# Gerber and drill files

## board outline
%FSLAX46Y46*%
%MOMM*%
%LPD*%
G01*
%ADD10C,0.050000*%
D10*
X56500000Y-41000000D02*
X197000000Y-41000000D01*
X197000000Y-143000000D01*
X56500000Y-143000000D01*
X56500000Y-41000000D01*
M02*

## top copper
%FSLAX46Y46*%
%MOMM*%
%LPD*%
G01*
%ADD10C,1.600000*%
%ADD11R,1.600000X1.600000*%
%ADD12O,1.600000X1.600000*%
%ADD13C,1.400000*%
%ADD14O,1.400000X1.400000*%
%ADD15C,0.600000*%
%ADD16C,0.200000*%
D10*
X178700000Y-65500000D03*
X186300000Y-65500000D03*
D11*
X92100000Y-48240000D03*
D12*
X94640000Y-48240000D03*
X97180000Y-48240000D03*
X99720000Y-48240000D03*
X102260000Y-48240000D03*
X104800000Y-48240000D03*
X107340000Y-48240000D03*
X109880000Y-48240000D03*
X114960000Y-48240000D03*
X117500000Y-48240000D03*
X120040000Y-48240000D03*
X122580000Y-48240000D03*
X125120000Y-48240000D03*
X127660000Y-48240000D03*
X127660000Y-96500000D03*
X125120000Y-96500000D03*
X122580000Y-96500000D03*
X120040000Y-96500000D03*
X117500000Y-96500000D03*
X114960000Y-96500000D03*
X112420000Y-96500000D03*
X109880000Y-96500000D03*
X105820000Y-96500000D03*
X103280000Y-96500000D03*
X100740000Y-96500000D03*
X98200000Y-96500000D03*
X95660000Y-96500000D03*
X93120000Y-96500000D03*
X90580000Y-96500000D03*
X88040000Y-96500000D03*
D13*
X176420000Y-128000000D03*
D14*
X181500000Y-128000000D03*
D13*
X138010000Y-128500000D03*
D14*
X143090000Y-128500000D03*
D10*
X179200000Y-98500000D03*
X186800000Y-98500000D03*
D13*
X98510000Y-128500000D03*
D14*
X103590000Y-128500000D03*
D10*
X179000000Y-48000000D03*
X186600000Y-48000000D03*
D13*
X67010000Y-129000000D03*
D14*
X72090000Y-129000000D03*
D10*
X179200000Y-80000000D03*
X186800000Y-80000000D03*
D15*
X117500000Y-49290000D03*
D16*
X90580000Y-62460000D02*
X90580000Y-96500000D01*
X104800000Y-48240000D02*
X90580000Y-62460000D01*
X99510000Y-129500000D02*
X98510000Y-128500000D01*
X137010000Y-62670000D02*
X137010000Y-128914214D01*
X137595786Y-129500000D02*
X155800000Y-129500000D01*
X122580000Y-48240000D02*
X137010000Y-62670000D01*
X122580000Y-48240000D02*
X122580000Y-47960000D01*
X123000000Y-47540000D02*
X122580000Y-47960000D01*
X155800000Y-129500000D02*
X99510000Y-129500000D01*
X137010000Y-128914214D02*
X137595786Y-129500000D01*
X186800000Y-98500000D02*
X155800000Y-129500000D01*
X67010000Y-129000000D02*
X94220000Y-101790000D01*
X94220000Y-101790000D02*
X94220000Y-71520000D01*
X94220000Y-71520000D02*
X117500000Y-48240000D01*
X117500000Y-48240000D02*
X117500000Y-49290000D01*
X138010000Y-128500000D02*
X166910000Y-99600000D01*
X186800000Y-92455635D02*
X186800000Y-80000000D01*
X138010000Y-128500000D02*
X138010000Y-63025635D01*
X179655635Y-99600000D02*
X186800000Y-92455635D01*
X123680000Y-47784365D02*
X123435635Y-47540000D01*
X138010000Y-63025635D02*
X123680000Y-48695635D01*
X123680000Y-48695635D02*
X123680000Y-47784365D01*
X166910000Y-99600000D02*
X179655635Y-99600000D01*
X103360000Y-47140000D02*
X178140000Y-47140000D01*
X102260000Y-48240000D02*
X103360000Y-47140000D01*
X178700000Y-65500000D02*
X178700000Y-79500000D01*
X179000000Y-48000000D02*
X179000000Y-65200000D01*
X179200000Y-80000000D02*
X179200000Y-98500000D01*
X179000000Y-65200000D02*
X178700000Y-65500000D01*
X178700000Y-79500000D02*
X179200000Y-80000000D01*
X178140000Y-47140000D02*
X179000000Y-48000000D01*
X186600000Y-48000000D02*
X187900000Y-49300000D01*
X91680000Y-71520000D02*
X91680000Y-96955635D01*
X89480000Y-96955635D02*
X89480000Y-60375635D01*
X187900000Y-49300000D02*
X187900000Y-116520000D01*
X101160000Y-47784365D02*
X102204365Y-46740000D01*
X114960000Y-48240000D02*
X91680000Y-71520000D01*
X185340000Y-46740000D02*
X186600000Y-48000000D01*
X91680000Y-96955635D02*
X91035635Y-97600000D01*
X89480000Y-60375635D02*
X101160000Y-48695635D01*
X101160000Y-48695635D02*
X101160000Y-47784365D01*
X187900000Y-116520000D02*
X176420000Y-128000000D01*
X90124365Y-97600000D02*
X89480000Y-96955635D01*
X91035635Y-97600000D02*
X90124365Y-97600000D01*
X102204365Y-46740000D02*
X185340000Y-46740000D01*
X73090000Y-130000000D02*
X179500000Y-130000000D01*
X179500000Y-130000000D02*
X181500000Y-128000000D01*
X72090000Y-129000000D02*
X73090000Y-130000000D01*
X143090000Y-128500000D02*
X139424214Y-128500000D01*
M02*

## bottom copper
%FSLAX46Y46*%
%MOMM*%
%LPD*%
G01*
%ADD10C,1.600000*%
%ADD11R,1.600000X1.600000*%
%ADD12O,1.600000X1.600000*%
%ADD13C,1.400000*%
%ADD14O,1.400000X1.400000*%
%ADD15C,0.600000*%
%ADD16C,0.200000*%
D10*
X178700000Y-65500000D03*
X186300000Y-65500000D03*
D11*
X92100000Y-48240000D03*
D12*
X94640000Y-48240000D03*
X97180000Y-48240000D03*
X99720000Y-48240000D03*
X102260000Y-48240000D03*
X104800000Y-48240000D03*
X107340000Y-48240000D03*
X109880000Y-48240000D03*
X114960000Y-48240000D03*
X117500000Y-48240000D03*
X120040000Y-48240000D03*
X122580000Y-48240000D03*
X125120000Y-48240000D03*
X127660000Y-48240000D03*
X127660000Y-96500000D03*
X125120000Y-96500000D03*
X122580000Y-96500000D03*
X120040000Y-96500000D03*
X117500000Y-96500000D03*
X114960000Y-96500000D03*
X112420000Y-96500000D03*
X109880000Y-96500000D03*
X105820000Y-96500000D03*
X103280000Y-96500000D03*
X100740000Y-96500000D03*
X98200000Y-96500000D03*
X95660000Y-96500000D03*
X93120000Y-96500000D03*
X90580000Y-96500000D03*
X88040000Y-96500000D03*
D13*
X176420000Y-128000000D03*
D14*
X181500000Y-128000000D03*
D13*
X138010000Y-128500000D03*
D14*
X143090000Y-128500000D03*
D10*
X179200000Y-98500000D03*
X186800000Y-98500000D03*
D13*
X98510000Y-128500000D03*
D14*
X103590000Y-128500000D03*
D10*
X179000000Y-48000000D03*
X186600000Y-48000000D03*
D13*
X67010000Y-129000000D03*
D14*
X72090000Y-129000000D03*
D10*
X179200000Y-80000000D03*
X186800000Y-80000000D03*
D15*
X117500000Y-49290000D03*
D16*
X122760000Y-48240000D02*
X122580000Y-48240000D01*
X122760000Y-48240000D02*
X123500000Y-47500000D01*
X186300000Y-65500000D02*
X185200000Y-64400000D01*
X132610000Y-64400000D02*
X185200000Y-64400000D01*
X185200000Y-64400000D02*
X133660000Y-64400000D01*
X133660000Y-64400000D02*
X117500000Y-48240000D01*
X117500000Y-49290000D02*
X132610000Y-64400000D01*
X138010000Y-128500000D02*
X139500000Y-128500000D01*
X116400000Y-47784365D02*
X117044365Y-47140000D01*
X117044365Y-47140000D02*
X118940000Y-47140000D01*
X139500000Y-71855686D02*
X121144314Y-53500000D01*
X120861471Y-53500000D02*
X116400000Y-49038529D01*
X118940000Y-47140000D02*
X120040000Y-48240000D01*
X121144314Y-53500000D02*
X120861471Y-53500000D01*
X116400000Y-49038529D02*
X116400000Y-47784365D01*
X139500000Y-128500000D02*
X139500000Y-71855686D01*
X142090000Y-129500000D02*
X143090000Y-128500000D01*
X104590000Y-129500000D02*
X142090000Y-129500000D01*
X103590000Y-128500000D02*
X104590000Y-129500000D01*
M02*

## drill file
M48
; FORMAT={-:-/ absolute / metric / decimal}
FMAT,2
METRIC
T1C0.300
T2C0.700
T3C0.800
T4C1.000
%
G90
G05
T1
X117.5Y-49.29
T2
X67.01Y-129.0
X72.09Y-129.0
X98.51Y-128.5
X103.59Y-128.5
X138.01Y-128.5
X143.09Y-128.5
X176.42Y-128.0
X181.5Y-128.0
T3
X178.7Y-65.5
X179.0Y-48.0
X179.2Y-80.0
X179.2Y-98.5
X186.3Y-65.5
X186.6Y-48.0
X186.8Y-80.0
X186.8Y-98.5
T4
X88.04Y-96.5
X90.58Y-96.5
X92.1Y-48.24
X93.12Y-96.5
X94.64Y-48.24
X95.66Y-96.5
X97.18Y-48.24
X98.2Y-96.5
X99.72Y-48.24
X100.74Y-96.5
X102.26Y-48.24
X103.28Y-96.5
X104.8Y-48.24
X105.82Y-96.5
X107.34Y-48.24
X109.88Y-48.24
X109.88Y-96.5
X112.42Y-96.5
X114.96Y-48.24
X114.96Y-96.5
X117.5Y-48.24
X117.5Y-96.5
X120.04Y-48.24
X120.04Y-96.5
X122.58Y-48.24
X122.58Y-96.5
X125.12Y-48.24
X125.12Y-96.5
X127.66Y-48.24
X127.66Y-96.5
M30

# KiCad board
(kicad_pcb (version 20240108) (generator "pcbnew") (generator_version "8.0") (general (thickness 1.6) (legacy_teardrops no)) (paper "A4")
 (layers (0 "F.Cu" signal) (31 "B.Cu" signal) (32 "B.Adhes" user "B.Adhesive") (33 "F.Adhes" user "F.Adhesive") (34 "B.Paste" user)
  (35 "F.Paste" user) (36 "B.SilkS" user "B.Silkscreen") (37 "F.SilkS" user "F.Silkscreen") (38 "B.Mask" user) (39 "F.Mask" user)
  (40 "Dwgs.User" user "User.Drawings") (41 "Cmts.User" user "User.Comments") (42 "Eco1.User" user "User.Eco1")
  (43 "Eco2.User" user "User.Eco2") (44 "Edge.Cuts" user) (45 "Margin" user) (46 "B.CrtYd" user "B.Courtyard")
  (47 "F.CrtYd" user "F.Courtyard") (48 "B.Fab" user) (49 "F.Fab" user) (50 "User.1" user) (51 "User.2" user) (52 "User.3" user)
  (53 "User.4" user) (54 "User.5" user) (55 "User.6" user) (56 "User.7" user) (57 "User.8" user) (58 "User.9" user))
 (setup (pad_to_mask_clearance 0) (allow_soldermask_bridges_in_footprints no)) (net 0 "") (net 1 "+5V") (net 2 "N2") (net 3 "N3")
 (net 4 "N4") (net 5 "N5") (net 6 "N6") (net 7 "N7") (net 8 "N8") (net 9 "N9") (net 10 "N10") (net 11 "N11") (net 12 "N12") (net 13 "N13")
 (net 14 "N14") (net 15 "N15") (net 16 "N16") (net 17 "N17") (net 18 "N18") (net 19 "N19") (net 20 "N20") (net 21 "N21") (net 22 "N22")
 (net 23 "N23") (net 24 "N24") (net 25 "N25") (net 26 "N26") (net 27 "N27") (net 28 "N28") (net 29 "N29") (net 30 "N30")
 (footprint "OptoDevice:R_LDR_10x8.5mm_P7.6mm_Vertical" (layer "F.Cu") (at 178.7 65.5)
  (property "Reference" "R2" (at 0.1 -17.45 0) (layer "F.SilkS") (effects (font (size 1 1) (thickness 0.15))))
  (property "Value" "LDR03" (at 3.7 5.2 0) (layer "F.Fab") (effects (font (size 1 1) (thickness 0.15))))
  (pad "1" thru_hole circle (at 0 0) (size 1.6 1.6) (drill 0.8) (layers "*.Cu" "*.Mask") (remove_unused_layers no) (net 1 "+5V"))
  (pad "2" thru_hole circle (at 7.6 0) (size 1.6 1.6) (drill 0.8) (layers "*.Cu" "*.Mask") (remove_unused_layers no) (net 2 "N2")))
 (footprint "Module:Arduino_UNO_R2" (layer "F.Cu") (at 92.1 48.24)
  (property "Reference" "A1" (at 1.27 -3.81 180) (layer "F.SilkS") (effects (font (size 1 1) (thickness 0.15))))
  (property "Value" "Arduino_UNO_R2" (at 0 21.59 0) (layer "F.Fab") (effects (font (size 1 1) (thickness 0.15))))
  (pad "1" thru_hole rect (at 0 0 90) (size 1.6 1.6) (drill 1) (layers "*.Cu" "*.Mask") (remove_unused_layers no) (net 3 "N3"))
  (pad "2" thru_hole oval (at 2.54 0 90) (size 1.6 1.6) (drill 1) (layers "*.Cu" "*.Mask") (remove_unused_layers no) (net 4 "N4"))
  (pad "3" thru_hole oval (at 5.08 0 90) (size 1.6 1.6) (drill 1) (layers "*.Cu" "*.Mask") (remove_unused_layers no) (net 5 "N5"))
  (pad "4" thru_hole oval (at 7.62 0 90) (size 1.6 1.6) (drill 1) (layers "*.Cu" "*.Mask") (remove_unused_layers no) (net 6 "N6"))
  (pad "5" thru_hole oval (at 10.16 0 90) (size 1.6 1.6) (drill 1) (layers "*.Cu" "*.Mask") (remove_unused_layers no) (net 1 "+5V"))
  (pad "6" thru_hole oval (at 12.7 0 90) (size 1.6 1.6) (drill 1) (layers "*.Cu" "*.Mask") (remove_unused_layers no) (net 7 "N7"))
  (pad "7" thru_hole oval (at 15.24 0 90) (size 1.6 1.6) (drill 1) (layers "*.Cu" "*.Mask") (remove_unused_layers no) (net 7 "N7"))
  (pad "8" thru_hole oval (at 17.78 0 90) (size 1.6 1.6) (drill 1) (layers "*.Cu" "*.Mask") (remove_unused_layers no) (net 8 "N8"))
  (pad "9" thru_hole oval (at 22.86 0 90) (size 1.6 1.6) (drill 1) (layers "*.Cu" "*.Mask") (remove_unused_layers no) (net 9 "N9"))
  (pad "10" thru_hole oval (at 25.4 0 90) (size 1.6 1.6) (drill 1) (layers "*.Cu" "*.Mask") (remove_unused_layers no) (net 2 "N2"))
  (pad "11" thru_hole oval (at 27.94 0 90) (size 1.6 1.6) (drill 1) (layers "*.Cu" "*.Mask") (remove_unused_layers no) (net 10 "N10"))
  (pad "12" thru_hole oval (at 30.48 0 90) (size 1.6 1.6) (drill 1) (layers "*.Cu" "*.Mask") (remove_unused_layers no) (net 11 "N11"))
  (pad "13" thru_hole oval (at 33.02 0 90) (size 1.6 1.6) (drill 1) (layers "*.Cu" "*.Mask") (remove_unused_layers no) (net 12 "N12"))
  (pad "14" thru_hole oval (at 35.56 0 90) (size 1.6 1.6) (drill 1) (layers "*.Cu" "*.Mask") (remove_unused_layers no) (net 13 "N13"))
  (pad "15" thru_hole oval (at 35.56 48.26 90) (size 1.6 1.6) (drill 1) (layers "*.Cu" "*.Mask") (remove_unused_layers no) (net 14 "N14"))
  (pad "16" thru_hole oval (at 33.02 48.26 90) (size 1.6 1.6) (drill 1) (layers "*.Cu" "*.Mask") (remove_unused_layers no) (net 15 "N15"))
  (pad "17" thru_hole oval (at 30.48 48.26 90) (size 1.6 1.6) (drill 1) (layers "*.Cu" "*.Mask") (remove_unused_layers no) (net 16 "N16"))
  (pad "18" thru_hole oval (at 27.94 48.26 90) (size 1.6 1.6) (drill 1) (layers "*.Cu" "*.Mask") (remove_unused_layers no) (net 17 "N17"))
  (pad "19" thru_hole oval (at 25.4 48.26 90) (size 1.6 1.6) (drill 1) (layers "*.Cu" "*.Mask") (remove_unused_layers no) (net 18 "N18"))
  (pad "20" thru_hole oval (at 22.86 48.26 90) (size 1.6 1.6) (drill 1) (layers "*.Cu" "*.Mask") (remove_unused_layers no) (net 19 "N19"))
  (pad "21" thru_hole oval (at 20.32 48.26 90) (size 1.6 1.6) (drill 1) (layers "*.Cu" "*.Mask") (remove_unused_layers no) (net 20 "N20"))
  (pad "22" thru_hole oval (at 17.78 48.26 90) (size 1.6 1.6) (drill 1) (layers "*.Cu" "*.Mask") (remove_unused_layers no) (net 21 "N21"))
  (pad "23" thru_hole oval (at 13.72 48.26 90) (size 1.6 1.6) (drill 1) (layers "*.Cu" "*.Mask") (remove_unused_layers no) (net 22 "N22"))
  (pad "24" thru_hole oval (at 11.18 48.26 90) (size 1.6 1.6) (drill 1) (layers "*.Cu" "*.Mask") (remove_unused_layers no) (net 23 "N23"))
  (pad "25" thru_hole oval (at 8.64 48.26 90) (size 1.6 1.6) (drill 1) (layers "*.Cu" "*.Mask") (remove_unused_layers no) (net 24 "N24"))
  (pad "26" thru_hole oval (at 6.1 48.26 90) (size 1.6 1.6) (drill 1) (layers "*.Cu" "*.Mask") (remove_unused_layers no) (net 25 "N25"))
  (pad "27" thru_hole oval (at 3.56 48.26 90) (size 1.6 1.6) (drill 1) (layers "*.Cu" "*.Mask") (remove_unused_layers no) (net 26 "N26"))
  (pad "28" thru_hole oval (at 1.02 48.26 90) (size 1.6 1.6) (drill 1) (layers "*.Cu" "*.Mask") (remove_unused_layers no) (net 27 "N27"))
  (pad "29" thru_hole oval (at -1.52 48.26 90) (size 1.6 1.6) (drill 1) (layers "*.Cu" "*.Mask") (remove_unused_layers no) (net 7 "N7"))
  (pad "30" thru_hole oval (at -4.06 48.26 90) (size 1.6 1.6) (drill 1) (layers "*.Cu" "*.Mask") (remove_unused_layers no) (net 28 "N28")))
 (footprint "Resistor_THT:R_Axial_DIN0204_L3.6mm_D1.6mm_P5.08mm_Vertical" (layer "F.Cu") (at 176.42 128)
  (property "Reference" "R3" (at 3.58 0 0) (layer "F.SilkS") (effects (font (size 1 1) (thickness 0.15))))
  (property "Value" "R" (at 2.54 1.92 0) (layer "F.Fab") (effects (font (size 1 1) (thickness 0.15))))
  (pad "1" thru_hole circle (at 0 0) (size 1.4 1.4) (drill 0.7) (layers "*.Cu" "*.Mask") (remove_unused_layers no) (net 9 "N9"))
  (pad "2" thru_hole oval (at 5.08 0) (size 1.4 1.4) (drill 0.7) (layers "*.Cu" "*.Mask") (remove_unused_layers no) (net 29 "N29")))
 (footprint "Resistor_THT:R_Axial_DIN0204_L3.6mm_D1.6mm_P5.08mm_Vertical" (layer "F.Cu") (at 138.01 128.5)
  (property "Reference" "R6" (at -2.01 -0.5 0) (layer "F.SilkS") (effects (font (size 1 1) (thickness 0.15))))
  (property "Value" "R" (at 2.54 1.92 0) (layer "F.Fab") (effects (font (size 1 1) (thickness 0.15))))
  (pad "1" thru_hole circle (at 0 0) (size 1.4 1.4) (drill 0.7) (layers "*.Cu" "*.Mask") (remove_unused_layers no) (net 10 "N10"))
  (pad "2" thru_hole oval (at 5.08 0) (size 1.4 1.4) (drill 0.7) (layers "*.Cu" "*.Mask") (remove_unused_layers no) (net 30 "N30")))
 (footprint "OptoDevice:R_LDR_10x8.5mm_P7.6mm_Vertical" (layer "F.Cu") (at 179.2 98.5)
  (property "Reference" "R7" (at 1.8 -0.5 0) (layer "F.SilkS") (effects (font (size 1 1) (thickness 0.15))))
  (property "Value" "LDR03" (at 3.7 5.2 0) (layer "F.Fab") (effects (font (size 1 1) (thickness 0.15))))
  (pad "1" thru_hole circle (at 0 0) (size 1.6 1.6) (drill 0.8) (layers "*.Cu" "*.Mask") (remove_unused_layers no) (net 1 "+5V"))
  (pad "2" thru_hole circle (at 7.6 0) (size 1.6 1.6) (drill 0.8) (layers "*.Cu" "*.Mask") (remove_unused_layers no) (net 11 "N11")))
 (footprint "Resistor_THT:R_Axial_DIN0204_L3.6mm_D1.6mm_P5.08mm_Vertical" (layer "F.Cu") (at 98.51 128.5)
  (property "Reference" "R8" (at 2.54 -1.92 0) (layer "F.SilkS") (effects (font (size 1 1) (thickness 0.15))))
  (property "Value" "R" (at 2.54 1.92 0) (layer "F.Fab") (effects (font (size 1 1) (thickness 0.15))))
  (pad "1" thru_hole circle (at 0 0) (size 1.4 1.4) (drill 0.7) (layers "*.Cu" "*.Mask") (remove_unused_layers no) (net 11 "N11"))
  (pad "2" thru_hole oval (at 5.08 0) (size 1.4 1.4) (drill 0.7) (layers "*.Cu" "*.Mask") (remove_unused_layers no) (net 30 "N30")))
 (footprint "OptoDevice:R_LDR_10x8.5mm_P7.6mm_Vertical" (layer "F.Cu") (at 179 48)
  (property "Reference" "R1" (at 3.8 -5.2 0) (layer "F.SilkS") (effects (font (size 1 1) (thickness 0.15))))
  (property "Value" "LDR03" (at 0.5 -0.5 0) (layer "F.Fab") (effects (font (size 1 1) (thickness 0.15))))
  (pad "1" thru_hole circle (at 0 0) (size 1.6 1.6) (drill 0.8) (layers "*.Cu" "*.Mask") (remove_unused_layers no) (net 1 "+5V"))
  (pad "2" thru_hole circle (at 7.6 0) (size 1.6 1.6) (drill 0.8) (layers "*.Cu" "*.Mask") (remove_unused_layers no) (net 9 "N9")))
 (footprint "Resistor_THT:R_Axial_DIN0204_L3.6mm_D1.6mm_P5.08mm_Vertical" (layer "F.Cu") (at 67.01 129)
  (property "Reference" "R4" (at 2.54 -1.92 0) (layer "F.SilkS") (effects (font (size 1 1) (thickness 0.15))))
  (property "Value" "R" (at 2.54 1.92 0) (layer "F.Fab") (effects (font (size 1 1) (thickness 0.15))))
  (pad "1" thru_hole circle (at 0 0) (size 1.4 1.4) (drill 0.7) (layers "*.Cu" "*.Mask") (remove_unused_layers no) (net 2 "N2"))
  (pad "2" thru_hole oval (at 5.08 0) (size 1.4 1.4) (drill 0.7) (layers "*.Cu" "*.Mask") (remove_unused_layers no) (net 29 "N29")))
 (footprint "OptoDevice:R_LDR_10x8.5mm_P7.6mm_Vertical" (layer "F.Cu") (at 179.2 80)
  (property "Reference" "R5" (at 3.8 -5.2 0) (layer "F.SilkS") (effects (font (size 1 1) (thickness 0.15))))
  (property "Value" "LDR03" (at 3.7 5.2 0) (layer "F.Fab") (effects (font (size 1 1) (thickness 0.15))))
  (pad "1" thru_hole circle (at 0 0) (size 1.6 1.6) (drill 0.8) (layers "*.Cu" "*.Mask") (remove_unused_layers no) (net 1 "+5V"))
  (pad "2" thru_hole circle (at 7.6 0) (size 1.6 1.6) (drill 0.8) (layers "*.Cu" "*.Mask") (remove_unused_layers no) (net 10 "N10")))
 (gr_rect (start 56.5 41) (end 197 143) (stroke (width 0.05) (type default)) (fill none) (layer "Edge.Cuts"))
 (segment (start 90.58 62.46) (end 90.58 96.5) (width 0.2) (layer "F.Cu") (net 7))
 (segment (start 104.8 48.24) (end 90.58 62.46) (width 0.2) (layer "F.Cu") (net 7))
 (segment (start 99.51 129.5) (end 98.51 128.5) (width 0.2) (layer "F.Cu") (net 11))
 (segment (start 137.01 62.67) (end 137.01 128.914214) (width 0.2) (layer "F.Cu") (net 11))
 (segment (start 137.595786 129.5) (end 155.8 129.5) (width 0.2) (layer "F.Cu") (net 11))
 (segment (start 122.58 48.24) (end 137.01 62.67) (width 0.2) (layer "F.Cu") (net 11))
 (segment (start 122.58 48.24) (end 122.58 47.96) (width 0.2) (layer "F.Cu") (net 11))
 (segment (start 123 47.54) (end 122.58 47.96) (width 0.2) (layer "F.Cu") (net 11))
 (segment (start 155.8 129.5) (end 99.51 129.5) (width 0.2) (layer "F.Cu") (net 11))
 (segment (start 137.01 128.914214) (end 137.595786 129.5) (width 0.2) (layer "F.Cu") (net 11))
 (segment (start 186.8 98.5) (end 155.8 129.5) (width 0.2) (layer "F.Cu") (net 11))
 (segment (start 122.76 48.24) (end 122.58 48.24) (width 0.2) (layer "B.Cu") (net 11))
 (segment (start 122.76 48.24) (end 123.5 47.5) (width 0.2) (layer "B.Cu") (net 11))
 (segment (start 67.01 129) (end 94.22 101.79) (width 0.2) (layer "F.Cu") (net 2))
 (segment (start 94.22 101.79) (end 94.22 71.52) (width 0.2) (layer "F.Cu") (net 2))
 (segment (start 94.22 71.52) (end 117.5 48.24) (width 0.2) (layer "F.Cu") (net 2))
 (segment (start 117.5 48.24) (end 117.5 49.29) (width 0.2) (layer "F.Cu") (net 2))
 (via (at 117.5 49.29) (size 0.6) (drill 0.3) (layers "F.Cu" "B.Cu") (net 2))
 (segment (start 186.3 65.5) (end 185.2 64.4) (width 0.2) (layer "B.Cu") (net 2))
 (segment (start 132.61 64.4) (end 185.2 64.4) (width 0.2) (layer "B.Cu") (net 2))
 (segment (start 185.2 64.4) (end 133.66 64.4) (width 0.2) (layer "B.Cu") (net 2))
 (segment (start 133.66 64.4) (end 117.5 48.24) (width 0.2) (layer "B.Cu") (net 2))
 (segment (start 117.5 49.29) (end 132.61 64.4) (width 0.2) (layer "B.Cu") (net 2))
 (segment (start 138.01 128.5) (end 166.91 99.6) (width 0.2) (layer "F.Cu") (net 10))
 (segment (start 186.8 92.455635) (end 186.8 80) (width 0.2) (layer "F.Cu") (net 10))
 (segment (start 138.01 128.5) (end 138.01 63.025635) (width 0.2) (layer "F.Cu") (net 10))
 (segment (start 179.655635 99.6) (end 186.8 92.455635) (width 0.2) (layer "F.Cu") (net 10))
 (segment (start 123.68 47.784365) (end 123.435635 47.54) (width 0.2) (layer "F.Cu") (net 10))
 (segment (start 138.01 63.025635) (end 123.68 48.695635) (width 0.2) (layer "F.Cu") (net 10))
 (segment (start 123.68 48.695635) (end 123.68 47.784365) (width 0.2) (layer "F.Cu") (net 10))
 (segment (start 166.91 99.6) (end 179.655635 99.6) (width 0.2) (layer "F.Cu") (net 10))
 (segment (start 138.01 128.5) (end 139.5 128.5) (width 0.2) (layer "B.Cu") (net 10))
 (segment (start 116.4 47.784365) (end 117.044365 47.14) (width 0.2) (layer "B.Cu") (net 10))
 (segment (start 117.044365 47.14) (end 118.94 47.14) (width 0.2) (layer "B.Cu") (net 10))
 (segment (start 139.5 71.855686) (end 121.144314 53.5) (width 0.2) (layer "B.Cu") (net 10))
 (segment (start 120.861471 53.5) (end 116.4 49.038529) (width 0.2) (layer "B.Cu") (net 10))
 (segment (start 118.94 47.14) (end 120.04 48.24) (width 0.2) (layer "B.Cu") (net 10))
 (segment (start 121.144314 53.5) (end 120.861471 53.5) (width 0.2) (layer "B.Cu") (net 10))
 (segment (start 116.4 49.038529) (end 116.4 47.784365) (width 0.2) (layer "B.Cu") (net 10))
 (segment (start 139.5 128.5) (end 139.5 71.855686) (width 0.2) (layer "B.Cu") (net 10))
 (segment (start 103.36 47.14) (end 178.14 47.14) (width 0.2) (layer "F.Cu") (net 1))
 (segment (start 102.26 48.24) (end 103.36 47.14) (width 0.2) (layer "F.Cu") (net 1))
 (segment (start 178.7 65.5) (end 178.7 79.5) (width 0.2) (layer "F.Cu") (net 1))
 (segment (start 179 48) (end 179 65.2) (width 0.2) (layer "F.Cu") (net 1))
 (segment (start 179.2 80) (end 179.2 98.5) (width 0.2) (layer "F.Cu") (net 1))
 (segment (start 179 65.2) (end 178.7 65.5) (width 0.2) (layer "F.Cu") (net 1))
 (segment (start 178.7 79.5) (end 179.2 80) (width 0.2) (layer "F.Cu") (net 1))
 (segment (start 178.14 47.14) (end 179 48) (width 0.2) (layer "F.Cu") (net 1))
 (segment (start 186.6 48) (end 187.9 49.3) (width 0.2) (layer "F.Cu") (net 9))
 (segment (start 91.68 71.52) (end 91.68 96.955635) (width 0.2) (layer "F.Cu") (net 9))
 (segment (start 89.48 96.955635) (end 89.48 60.375635) (width 0.2) (layer "F.Cu") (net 9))
 (segment (start 187.9 49.3) (end 187.9 116.52) (width 0.2) (layer "F.Cu") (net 9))
 (segment (start 101.16 47.784365) (end 102.204365 46.74) (width 0.2) (layer "F.Cu") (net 9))
 (segment (start 114.96 48.24) (end 91.68 71.52) (width 0.2) (layer "F.Cu") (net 9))
 (segment (start 185.34 46.74) (end 186.6 48) (width 0.2) (layer "F.Cu") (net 9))
 (segment (start 91.68 96.955635) (end 91.035635 97.6) (width 0.2) (layer "F.Cu") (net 9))
 (segment (start 89.48 60.375635) (end 101.16 48.695635) (width 0.2) (layer "F.Cu") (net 9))
 (segment (start 101.16 48.695635) (end 101.16 47.784365) (width 0.2) (layer "F.Cu") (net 9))
 (segment (start 187.9 116.52) (end 176.42 128) (width 0.2) (layer "F.Cu") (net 9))
 (segment (start 90.124365 97.6) (end 89.48 96.955635) (width 0.2) (layer "F.Cu") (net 9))
 (segment (start 91.035635 97.6) (end 90.124365 97.6) (width 0.2) (layer "F.Cu") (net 9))
 (segment (start 102.204365 46.74) (end 185.34 46.74) (width 0.2) (layer "F.Cu") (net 9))
 (segment (start 73.09 130) (end 179.5 130) (width 0.2) (layer "F.Cu") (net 29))
 (segment (start 179.5 130) (end 181.5 128) (width 0.2) (layer "F.Cu") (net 29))
 (segment (start 72.09 129) (end 73.09 130) (width 0.2) (layer "F.Cu") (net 29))
 (segment (start 143.09 128.5) (end 139.424214 128.5) (width 0.2) (layer "F.Cu") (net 30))
 (segment (start 142.09 129.5) (end 143.09 128.5) (width 0.2) (layer "B.Cu") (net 30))
 (segment (start 104.59 129.5) (end 142.09 129.5) (width 0.2) (layer "B.Cu") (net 30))
 (segment (start 103.59 128.5) (end 104.59 129.5) (width 0.2) (layer "B.Cu") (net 30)))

